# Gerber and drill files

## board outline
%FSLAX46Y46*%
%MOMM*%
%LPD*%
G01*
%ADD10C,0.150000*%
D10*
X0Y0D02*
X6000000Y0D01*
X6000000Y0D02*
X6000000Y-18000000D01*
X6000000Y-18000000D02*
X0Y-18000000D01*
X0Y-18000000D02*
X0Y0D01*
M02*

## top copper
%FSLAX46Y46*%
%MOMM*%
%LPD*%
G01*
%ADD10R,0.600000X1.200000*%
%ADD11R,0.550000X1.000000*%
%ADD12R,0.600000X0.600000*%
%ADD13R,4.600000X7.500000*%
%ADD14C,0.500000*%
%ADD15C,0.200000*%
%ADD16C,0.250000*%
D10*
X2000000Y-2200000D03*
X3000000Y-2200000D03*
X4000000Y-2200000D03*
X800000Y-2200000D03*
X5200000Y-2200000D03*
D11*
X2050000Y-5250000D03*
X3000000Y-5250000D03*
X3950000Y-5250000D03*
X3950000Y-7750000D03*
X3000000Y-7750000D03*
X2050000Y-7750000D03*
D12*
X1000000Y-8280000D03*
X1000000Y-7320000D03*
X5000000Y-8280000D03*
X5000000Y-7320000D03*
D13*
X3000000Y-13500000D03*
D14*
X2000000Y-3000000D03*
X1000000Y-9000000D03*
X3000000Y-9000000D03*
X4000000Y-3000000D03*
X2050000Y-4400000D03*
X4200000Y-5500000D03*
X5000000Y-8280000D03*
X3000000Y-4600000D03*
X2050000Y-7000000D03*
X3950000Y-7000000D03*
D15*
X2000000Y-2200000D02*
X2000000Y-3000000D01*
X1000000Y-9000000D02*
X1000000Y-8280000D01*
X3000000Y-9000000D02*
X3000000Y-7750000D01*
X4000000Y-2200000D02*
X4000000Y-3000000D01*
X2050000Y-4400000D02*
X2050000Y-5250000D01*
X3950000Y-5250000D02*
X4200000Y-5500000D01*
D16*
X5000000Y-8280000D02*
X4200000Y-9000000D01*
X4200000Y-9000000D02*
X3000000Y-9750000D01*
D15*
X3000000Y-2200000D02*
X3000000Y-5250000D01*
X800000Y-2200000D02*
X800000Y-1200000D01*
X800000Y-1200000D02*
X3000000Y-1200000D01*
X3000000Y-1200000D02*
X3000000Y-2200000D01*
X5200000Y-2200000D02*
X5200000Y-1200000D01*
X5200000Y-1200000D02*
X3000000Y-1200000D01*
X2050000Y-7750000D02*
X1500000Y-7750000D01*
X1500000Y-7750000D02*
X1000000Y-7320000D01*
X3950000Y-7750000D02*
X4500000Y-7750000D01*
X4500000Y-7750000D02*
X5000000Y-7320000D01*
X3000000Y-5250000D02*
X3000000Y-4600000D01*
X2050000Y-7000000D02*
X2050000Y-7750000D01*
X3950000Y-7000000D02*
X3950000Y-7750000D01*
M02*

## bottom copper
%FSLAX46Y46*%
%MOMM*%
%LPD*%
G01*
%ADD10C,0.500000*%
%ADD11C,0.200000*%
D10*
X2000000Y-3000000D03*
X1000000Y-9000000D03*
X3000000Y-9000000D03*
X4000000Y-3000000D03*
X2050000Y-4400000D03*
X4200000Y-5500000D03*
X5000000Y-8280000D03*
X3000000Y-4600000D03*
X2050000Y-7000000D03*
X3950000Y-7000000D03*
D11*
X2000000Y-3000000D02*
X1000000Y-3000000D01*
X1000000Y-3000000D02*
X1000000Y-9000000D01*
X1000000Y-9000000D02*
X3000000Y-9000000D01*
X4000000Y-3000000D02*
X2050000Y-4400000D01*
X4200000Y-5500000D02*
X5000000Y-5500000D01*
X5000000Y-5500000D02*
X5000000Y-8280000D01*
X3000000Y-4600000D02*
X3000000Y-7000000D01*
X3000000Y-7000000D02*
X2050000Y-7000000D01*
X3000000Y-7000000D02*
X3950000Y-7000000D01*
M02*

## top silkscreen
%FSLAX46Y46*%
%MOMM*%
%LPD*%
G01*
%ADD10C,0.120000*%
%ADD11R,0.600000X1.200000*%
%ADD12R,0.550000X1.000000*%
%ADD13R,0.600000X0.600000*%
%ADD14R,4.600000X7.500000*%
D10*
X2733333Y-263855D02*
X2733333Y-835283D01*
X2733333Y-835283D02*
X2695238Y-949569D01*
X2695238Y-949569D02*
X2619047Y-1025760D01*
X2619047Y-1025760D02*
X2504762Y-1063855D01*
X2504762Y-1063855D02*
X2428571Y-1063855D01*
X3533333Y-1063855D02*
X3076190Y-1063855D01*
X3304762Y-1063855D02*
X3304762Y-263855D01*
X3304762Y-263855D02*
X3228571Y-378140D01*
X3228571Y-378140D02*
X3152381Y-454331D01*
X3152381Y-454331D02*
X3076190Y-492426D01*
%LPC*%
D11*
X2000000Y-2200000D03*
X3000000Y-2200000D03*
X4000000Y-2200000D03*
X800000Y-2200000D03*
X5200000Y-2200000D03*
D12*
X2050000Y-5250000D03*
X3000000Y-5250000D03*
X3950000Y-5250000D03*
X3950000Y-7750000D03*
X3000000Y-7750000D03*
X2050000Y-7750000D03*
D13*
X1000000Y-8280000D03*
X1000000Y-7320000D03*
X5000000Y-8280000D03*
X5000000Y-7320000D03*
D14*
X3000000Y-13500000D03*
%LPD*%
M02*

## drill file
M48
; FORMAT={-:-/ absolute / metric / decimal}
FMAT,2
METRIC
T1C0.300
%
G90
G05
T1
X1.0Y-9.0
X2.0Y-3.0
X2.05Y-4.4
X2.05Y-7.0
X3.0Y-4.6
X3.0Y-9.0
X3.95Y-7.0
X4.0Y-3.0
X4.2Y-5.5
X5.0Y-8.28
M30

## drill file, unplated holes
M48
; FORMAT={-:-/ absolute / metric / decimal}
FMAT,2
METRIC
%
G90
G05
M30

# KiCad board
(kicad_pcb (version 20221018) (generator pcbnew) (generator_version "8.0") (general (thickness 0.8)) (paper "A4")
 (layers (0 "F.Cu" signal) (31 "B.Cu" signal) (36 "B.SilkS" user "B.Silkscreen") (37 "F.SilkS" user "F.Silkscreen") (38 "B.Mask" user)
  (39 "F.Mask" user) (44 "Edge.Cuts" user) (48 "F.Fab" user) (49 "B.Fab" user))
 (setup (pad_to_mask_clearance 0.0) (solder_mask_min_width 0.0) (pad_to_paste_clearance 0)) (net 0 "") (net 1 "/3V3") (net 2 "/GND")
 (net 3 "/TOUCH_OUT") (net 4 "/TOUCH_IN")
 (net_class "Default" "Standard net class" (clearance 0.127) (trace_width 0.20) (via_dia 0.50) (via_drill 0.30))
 (gr_line (start 0 0) (end 6.0 0) (layer "Edge.Cuts") (width 0.15))
 (gr_line (start 6.0 0) (end 6.0 18.0) (layer "Edge.Cuts") (width 0.15))
 (gr_line (start 6.0 18.0) (end 0 18.0) (layer "Edge.Cuts") (width 0.15))
 (gr_line (start 0 18.0) (end 0 0) (layer "Edge.Cuts") (width 0.15))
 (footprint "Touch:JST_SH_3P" (layer "F.Cu") (at 3.0 2.2)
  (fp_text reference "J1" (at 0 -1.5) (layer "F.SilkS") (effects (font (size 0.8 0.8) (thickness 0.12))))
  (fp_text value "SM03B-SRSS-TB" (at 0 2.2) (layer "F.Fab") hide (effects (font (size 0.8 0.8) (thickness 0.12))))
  (pad "1" smd rect (at -1.0 0) (size 0.6 1.2) (layers "F.Cu" "F.Paste" "F.Mask") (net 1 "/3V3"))
  (pad "2" smd rect (at 0.0 0) (size 0.6 1.2) (layers "F.Cu" "F.Paste" "F.Mask") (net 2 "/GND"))
  (pad "3" smd rect (at 1.0 0) (size 0.6 1.2) (layers "F.Cu" "F.Paste" "F.Mask") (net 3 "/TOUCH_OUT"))
  (pad "4" smd rect (at -2.2 0) (size 0.6 1.2) (layers "F.Cu" "F.Paste" "F.Mask") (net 2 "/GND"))
  (pad "4" smd rect (at 2.2 0) (size 0.6 1.2) (layers "F.Cu" "F.Paste" "F.Mask") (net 2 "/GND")))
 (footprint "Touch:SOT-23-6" (layer "F.Cu") (at 3.0 6.5)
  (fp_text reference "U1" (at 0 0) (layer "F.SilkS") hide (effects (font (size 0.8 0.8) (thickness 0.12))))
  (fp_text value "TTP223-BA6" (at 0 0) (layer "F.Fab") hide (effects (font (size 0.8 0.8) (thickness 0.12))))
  (pad "1" smd rect (at -0.95 -1.25) (size 0.55 1.0) (layers "F.Cu" "F.Paste" "F.Mask") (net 3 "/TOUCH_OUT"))
  (pad "2" smd rect (at 0.0 -1.25) (size 0.55 1.0) (layers "F.Cu" "F.Paste" "F.Mask") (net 2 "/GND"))
  (pad "3" smd rect (at 0.95 -1.25) (size 0.55 1.0) (layers "F.Cu" "F.Paste" "F.Mask") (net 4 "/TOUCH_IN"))
  (pad "4" smd rect (at 0.95 1.25) (size 0.55 1.0) (layers "F.Cu" "F.Paste" "F.Mask") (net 2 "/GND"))
  (pad "5" smd rect (at 0.0 1.25) (size 0.55 1.0) (layers "F.Cu" "F.Paste" "F.Mask") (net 1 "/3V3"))
  (pad "6" smd rect (at -0.95 1.25) (size 0.55 1.0) (layers "F.Cu" "F.Paste" "F.Mask") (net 2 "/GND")))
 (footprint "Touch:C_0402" (layer "F.Cu") (at 1.0 7.8 90)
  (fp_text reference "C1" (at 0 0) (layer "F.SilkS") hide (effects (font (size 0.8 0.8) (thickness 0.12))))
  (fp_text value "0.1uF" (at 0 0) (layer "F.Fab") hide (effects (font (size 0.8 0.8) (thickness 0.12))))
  (pad "1" smd rect (at -0.48 0 90) (size 0.6 0.6) (layers "F.Cu" "F.Paste" "F.Mask") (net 1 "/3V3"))
  (pad "2" smd rect (at 0.48 0 90) (size 0.6 0.6) (layers "F.Cu" "F.Paste" "F.Mask") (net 2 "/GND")))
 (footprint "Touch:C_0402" (layer "F.Cu") (at 5.0 7.8 90)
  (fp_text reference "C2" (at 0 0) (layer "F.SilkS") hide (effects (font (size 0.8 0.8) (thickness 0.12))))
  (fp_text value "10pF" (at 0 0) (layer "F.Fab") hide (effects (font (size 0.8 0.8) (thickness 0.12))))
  (pad "1" smd rect (at -0.48 0 90) (size 0.6 0.6) (layers "F.Cu" "F.Paste" "F.Mask") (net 4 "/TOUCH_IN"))
  (pad "2" smd rect (at 0.48 0 90) (size 0.6 0.6) (layers "F.Cu" "F.Paste" "F.Mask") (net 2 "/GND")))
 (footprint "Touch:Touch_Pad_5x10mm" (layer "F.Cu") (at 3.0 13.5)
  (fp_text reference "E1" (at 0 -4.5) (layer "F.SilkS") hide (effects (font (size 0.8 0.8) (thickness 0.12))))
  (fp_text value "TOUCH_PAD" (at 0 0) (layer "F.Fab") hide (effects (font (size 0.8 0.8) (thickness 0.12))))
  (pad "1" smd rect (at 0 0) (size 4.6 7.5) (layers "F.Cu" "F.Paste" "F.Mask") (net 4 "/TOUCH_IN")))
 (segment (start 2.0 2.2) (end 2.0 3.0) (width 0.20) (layer "F.Cu") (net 1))
 (via (at 2.0 3.0) (size 0.5) (drill 0.3) (layers "F.Cu" "B.Cu") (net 1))
 (segment (start 2.0 3.0) (end 1.0 3.0) (width 0.20) (layer "B.Cu") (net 1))
 (segment (start 1.0 3.0) (end 1.0 9.0) (width 0.20) (layer "B.Cu") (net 1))
 (via (at 1.0 9.0) (size 0.5) (drill 0.3) (layers "F.Cu" "B.Cu") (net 1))
 (segment (start 1.0 9.0) (end 1.0 8.28) (width 0.20) (layer "F.Cu") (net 1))
 (segment (start 1.0 9.0) (end 3.0 9.0) (width 0.20) (layer "B.Cu") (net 1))
 (via (at 3.0 9.0) (size 0.5) (drill 0.3) (layers "F.Cu" "B.Cu") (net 1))
 (segment (start 3.0 9.0) (end 3.0 7.75) (width 0.20) (layer "F.Cu") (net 1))
 (segment (start 4.0 2.2) (end 4.0 3.0) (width 0.20) (layer "F.Cu") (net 3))
 (via (at 4.0 3.0) (size 0.5) (drill 0.3) (layers "F.Cu" "B.Cu") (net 3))
 (segment (start 4.0 3.0) (end 2.05 4.4) (width 0.20) (layer "B.Cu") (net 3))
 (via (at 2.05 4.4) (size 0.5) (drill 0.3) (layers "F.Cu" "B.Cu") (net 3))
 (segment (start 2.05 4.4) (end 2.05 5.25) (width 0.20) (layer "F.Cu") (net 3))
 (segment (start 3.95 5.25) (end 4.2 5.5) (width 0.20) (layer "F.Cu") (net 4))
 (via (at 4.2 5.5) (size 0.5) (drill 0.3) (layers "F.Cu" "B.Cu") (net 4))
 (segment (start 4.2 5.5) (end 5.0 5.5) (width 0.20) (layer "B.Cu") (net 4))
 (segment (start 5.0 5.5) (end 5.0 8.28) (width 0.20) (layer "B.Cu") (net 4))
 (via (at 5.0 8.28) (size 0.5) (drill 0.3) (layers "F.Cu" "B.Cu") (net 4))
 (segment (start 5.0 8.28) (end 4.2 9.0) (width 0.25) (layer "F.Cu") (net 4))
 (segment (start 4.2 9.0) (end 3.0 9.75) (width 0.25) (layer "F.Cu") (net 4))
 (segment (start 3.0 2.2) (end 3.0 5.25) (width 0.20) (layer "F.Cu") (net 2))
 (segment (start 0.8 2.2) (end 0.8 1.2) (width 0.20) (layer "F.Cu") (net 2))
 (segment (start 0.8 1.2) (end 3.0 1.2) (width 0.20) (layer "F.Cu") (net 2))
 (segment (start 3.0 1.2) (end 3.0 2.2) (width 0.20) (layer "F.Cu") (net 2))
 (segment (start 5.2 2.2) (end 5.2 1.2) (width 0.20) (layer "F.Cu") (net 2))
 (segment (start 5.2 1.2) (end 3.0 1.2) (width 0.20) (layer "F.Cu") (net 2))
 (segment (start 2.05 7.75) (end 1.5 7.75) (width 0.20) (layer "F.Cu") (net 2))
 (segment (start 1.5 7.75) (end 1.0 7.32) (width 0.20) (layer "F.Cu") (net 2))
 (segment (start 3.95 7.75) (end 4.5 7.75) (width 0.20) (layer "F.Cu") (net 2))
 (segment (start 4.5 7.75) (end 5.0 7.32) (width 0.20) (layer "F.Cu") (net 2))
 (via (at 3.0 4.6) (size 0.5) (drill 0.3) (layers "F.Cu" "B.Cu") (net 2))
 (segment (start 3.0 5.25) (end 3.0 4.6) (width 0.20) (layer "F.Cu") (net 2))
 (segment (start 3.0 4.6) (end 3.0 7.0) (width 0.20) (layer "B.Cu") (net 2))
 (segment (start 3.0 7.0) (end 2.05 7.0) (width 0.20) (layer "B.Cu") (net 2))
 (via (at 2.05 7.0) (size 0.5) (drill 0.3) (layers "F.Cu" "B.Cu") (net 2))
 (segment (start 2.05 7.0) (end 2.05 7.75) (width 0.20) (layer "F.Cu") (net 2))
 (segment (start 3.0 7.0) (end 3.95 7.0) (width 0.20) (layer "B.Cu") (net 2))
 (via (at 3.95 7.0) (size 0.5) (drill 0.3) (layers "F.Cu" "B.Cu") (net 2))
 (segment (start 3.95 7.0) (end 3.95 7.75) (width 0.20) (layer "F.Cu") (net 2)))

